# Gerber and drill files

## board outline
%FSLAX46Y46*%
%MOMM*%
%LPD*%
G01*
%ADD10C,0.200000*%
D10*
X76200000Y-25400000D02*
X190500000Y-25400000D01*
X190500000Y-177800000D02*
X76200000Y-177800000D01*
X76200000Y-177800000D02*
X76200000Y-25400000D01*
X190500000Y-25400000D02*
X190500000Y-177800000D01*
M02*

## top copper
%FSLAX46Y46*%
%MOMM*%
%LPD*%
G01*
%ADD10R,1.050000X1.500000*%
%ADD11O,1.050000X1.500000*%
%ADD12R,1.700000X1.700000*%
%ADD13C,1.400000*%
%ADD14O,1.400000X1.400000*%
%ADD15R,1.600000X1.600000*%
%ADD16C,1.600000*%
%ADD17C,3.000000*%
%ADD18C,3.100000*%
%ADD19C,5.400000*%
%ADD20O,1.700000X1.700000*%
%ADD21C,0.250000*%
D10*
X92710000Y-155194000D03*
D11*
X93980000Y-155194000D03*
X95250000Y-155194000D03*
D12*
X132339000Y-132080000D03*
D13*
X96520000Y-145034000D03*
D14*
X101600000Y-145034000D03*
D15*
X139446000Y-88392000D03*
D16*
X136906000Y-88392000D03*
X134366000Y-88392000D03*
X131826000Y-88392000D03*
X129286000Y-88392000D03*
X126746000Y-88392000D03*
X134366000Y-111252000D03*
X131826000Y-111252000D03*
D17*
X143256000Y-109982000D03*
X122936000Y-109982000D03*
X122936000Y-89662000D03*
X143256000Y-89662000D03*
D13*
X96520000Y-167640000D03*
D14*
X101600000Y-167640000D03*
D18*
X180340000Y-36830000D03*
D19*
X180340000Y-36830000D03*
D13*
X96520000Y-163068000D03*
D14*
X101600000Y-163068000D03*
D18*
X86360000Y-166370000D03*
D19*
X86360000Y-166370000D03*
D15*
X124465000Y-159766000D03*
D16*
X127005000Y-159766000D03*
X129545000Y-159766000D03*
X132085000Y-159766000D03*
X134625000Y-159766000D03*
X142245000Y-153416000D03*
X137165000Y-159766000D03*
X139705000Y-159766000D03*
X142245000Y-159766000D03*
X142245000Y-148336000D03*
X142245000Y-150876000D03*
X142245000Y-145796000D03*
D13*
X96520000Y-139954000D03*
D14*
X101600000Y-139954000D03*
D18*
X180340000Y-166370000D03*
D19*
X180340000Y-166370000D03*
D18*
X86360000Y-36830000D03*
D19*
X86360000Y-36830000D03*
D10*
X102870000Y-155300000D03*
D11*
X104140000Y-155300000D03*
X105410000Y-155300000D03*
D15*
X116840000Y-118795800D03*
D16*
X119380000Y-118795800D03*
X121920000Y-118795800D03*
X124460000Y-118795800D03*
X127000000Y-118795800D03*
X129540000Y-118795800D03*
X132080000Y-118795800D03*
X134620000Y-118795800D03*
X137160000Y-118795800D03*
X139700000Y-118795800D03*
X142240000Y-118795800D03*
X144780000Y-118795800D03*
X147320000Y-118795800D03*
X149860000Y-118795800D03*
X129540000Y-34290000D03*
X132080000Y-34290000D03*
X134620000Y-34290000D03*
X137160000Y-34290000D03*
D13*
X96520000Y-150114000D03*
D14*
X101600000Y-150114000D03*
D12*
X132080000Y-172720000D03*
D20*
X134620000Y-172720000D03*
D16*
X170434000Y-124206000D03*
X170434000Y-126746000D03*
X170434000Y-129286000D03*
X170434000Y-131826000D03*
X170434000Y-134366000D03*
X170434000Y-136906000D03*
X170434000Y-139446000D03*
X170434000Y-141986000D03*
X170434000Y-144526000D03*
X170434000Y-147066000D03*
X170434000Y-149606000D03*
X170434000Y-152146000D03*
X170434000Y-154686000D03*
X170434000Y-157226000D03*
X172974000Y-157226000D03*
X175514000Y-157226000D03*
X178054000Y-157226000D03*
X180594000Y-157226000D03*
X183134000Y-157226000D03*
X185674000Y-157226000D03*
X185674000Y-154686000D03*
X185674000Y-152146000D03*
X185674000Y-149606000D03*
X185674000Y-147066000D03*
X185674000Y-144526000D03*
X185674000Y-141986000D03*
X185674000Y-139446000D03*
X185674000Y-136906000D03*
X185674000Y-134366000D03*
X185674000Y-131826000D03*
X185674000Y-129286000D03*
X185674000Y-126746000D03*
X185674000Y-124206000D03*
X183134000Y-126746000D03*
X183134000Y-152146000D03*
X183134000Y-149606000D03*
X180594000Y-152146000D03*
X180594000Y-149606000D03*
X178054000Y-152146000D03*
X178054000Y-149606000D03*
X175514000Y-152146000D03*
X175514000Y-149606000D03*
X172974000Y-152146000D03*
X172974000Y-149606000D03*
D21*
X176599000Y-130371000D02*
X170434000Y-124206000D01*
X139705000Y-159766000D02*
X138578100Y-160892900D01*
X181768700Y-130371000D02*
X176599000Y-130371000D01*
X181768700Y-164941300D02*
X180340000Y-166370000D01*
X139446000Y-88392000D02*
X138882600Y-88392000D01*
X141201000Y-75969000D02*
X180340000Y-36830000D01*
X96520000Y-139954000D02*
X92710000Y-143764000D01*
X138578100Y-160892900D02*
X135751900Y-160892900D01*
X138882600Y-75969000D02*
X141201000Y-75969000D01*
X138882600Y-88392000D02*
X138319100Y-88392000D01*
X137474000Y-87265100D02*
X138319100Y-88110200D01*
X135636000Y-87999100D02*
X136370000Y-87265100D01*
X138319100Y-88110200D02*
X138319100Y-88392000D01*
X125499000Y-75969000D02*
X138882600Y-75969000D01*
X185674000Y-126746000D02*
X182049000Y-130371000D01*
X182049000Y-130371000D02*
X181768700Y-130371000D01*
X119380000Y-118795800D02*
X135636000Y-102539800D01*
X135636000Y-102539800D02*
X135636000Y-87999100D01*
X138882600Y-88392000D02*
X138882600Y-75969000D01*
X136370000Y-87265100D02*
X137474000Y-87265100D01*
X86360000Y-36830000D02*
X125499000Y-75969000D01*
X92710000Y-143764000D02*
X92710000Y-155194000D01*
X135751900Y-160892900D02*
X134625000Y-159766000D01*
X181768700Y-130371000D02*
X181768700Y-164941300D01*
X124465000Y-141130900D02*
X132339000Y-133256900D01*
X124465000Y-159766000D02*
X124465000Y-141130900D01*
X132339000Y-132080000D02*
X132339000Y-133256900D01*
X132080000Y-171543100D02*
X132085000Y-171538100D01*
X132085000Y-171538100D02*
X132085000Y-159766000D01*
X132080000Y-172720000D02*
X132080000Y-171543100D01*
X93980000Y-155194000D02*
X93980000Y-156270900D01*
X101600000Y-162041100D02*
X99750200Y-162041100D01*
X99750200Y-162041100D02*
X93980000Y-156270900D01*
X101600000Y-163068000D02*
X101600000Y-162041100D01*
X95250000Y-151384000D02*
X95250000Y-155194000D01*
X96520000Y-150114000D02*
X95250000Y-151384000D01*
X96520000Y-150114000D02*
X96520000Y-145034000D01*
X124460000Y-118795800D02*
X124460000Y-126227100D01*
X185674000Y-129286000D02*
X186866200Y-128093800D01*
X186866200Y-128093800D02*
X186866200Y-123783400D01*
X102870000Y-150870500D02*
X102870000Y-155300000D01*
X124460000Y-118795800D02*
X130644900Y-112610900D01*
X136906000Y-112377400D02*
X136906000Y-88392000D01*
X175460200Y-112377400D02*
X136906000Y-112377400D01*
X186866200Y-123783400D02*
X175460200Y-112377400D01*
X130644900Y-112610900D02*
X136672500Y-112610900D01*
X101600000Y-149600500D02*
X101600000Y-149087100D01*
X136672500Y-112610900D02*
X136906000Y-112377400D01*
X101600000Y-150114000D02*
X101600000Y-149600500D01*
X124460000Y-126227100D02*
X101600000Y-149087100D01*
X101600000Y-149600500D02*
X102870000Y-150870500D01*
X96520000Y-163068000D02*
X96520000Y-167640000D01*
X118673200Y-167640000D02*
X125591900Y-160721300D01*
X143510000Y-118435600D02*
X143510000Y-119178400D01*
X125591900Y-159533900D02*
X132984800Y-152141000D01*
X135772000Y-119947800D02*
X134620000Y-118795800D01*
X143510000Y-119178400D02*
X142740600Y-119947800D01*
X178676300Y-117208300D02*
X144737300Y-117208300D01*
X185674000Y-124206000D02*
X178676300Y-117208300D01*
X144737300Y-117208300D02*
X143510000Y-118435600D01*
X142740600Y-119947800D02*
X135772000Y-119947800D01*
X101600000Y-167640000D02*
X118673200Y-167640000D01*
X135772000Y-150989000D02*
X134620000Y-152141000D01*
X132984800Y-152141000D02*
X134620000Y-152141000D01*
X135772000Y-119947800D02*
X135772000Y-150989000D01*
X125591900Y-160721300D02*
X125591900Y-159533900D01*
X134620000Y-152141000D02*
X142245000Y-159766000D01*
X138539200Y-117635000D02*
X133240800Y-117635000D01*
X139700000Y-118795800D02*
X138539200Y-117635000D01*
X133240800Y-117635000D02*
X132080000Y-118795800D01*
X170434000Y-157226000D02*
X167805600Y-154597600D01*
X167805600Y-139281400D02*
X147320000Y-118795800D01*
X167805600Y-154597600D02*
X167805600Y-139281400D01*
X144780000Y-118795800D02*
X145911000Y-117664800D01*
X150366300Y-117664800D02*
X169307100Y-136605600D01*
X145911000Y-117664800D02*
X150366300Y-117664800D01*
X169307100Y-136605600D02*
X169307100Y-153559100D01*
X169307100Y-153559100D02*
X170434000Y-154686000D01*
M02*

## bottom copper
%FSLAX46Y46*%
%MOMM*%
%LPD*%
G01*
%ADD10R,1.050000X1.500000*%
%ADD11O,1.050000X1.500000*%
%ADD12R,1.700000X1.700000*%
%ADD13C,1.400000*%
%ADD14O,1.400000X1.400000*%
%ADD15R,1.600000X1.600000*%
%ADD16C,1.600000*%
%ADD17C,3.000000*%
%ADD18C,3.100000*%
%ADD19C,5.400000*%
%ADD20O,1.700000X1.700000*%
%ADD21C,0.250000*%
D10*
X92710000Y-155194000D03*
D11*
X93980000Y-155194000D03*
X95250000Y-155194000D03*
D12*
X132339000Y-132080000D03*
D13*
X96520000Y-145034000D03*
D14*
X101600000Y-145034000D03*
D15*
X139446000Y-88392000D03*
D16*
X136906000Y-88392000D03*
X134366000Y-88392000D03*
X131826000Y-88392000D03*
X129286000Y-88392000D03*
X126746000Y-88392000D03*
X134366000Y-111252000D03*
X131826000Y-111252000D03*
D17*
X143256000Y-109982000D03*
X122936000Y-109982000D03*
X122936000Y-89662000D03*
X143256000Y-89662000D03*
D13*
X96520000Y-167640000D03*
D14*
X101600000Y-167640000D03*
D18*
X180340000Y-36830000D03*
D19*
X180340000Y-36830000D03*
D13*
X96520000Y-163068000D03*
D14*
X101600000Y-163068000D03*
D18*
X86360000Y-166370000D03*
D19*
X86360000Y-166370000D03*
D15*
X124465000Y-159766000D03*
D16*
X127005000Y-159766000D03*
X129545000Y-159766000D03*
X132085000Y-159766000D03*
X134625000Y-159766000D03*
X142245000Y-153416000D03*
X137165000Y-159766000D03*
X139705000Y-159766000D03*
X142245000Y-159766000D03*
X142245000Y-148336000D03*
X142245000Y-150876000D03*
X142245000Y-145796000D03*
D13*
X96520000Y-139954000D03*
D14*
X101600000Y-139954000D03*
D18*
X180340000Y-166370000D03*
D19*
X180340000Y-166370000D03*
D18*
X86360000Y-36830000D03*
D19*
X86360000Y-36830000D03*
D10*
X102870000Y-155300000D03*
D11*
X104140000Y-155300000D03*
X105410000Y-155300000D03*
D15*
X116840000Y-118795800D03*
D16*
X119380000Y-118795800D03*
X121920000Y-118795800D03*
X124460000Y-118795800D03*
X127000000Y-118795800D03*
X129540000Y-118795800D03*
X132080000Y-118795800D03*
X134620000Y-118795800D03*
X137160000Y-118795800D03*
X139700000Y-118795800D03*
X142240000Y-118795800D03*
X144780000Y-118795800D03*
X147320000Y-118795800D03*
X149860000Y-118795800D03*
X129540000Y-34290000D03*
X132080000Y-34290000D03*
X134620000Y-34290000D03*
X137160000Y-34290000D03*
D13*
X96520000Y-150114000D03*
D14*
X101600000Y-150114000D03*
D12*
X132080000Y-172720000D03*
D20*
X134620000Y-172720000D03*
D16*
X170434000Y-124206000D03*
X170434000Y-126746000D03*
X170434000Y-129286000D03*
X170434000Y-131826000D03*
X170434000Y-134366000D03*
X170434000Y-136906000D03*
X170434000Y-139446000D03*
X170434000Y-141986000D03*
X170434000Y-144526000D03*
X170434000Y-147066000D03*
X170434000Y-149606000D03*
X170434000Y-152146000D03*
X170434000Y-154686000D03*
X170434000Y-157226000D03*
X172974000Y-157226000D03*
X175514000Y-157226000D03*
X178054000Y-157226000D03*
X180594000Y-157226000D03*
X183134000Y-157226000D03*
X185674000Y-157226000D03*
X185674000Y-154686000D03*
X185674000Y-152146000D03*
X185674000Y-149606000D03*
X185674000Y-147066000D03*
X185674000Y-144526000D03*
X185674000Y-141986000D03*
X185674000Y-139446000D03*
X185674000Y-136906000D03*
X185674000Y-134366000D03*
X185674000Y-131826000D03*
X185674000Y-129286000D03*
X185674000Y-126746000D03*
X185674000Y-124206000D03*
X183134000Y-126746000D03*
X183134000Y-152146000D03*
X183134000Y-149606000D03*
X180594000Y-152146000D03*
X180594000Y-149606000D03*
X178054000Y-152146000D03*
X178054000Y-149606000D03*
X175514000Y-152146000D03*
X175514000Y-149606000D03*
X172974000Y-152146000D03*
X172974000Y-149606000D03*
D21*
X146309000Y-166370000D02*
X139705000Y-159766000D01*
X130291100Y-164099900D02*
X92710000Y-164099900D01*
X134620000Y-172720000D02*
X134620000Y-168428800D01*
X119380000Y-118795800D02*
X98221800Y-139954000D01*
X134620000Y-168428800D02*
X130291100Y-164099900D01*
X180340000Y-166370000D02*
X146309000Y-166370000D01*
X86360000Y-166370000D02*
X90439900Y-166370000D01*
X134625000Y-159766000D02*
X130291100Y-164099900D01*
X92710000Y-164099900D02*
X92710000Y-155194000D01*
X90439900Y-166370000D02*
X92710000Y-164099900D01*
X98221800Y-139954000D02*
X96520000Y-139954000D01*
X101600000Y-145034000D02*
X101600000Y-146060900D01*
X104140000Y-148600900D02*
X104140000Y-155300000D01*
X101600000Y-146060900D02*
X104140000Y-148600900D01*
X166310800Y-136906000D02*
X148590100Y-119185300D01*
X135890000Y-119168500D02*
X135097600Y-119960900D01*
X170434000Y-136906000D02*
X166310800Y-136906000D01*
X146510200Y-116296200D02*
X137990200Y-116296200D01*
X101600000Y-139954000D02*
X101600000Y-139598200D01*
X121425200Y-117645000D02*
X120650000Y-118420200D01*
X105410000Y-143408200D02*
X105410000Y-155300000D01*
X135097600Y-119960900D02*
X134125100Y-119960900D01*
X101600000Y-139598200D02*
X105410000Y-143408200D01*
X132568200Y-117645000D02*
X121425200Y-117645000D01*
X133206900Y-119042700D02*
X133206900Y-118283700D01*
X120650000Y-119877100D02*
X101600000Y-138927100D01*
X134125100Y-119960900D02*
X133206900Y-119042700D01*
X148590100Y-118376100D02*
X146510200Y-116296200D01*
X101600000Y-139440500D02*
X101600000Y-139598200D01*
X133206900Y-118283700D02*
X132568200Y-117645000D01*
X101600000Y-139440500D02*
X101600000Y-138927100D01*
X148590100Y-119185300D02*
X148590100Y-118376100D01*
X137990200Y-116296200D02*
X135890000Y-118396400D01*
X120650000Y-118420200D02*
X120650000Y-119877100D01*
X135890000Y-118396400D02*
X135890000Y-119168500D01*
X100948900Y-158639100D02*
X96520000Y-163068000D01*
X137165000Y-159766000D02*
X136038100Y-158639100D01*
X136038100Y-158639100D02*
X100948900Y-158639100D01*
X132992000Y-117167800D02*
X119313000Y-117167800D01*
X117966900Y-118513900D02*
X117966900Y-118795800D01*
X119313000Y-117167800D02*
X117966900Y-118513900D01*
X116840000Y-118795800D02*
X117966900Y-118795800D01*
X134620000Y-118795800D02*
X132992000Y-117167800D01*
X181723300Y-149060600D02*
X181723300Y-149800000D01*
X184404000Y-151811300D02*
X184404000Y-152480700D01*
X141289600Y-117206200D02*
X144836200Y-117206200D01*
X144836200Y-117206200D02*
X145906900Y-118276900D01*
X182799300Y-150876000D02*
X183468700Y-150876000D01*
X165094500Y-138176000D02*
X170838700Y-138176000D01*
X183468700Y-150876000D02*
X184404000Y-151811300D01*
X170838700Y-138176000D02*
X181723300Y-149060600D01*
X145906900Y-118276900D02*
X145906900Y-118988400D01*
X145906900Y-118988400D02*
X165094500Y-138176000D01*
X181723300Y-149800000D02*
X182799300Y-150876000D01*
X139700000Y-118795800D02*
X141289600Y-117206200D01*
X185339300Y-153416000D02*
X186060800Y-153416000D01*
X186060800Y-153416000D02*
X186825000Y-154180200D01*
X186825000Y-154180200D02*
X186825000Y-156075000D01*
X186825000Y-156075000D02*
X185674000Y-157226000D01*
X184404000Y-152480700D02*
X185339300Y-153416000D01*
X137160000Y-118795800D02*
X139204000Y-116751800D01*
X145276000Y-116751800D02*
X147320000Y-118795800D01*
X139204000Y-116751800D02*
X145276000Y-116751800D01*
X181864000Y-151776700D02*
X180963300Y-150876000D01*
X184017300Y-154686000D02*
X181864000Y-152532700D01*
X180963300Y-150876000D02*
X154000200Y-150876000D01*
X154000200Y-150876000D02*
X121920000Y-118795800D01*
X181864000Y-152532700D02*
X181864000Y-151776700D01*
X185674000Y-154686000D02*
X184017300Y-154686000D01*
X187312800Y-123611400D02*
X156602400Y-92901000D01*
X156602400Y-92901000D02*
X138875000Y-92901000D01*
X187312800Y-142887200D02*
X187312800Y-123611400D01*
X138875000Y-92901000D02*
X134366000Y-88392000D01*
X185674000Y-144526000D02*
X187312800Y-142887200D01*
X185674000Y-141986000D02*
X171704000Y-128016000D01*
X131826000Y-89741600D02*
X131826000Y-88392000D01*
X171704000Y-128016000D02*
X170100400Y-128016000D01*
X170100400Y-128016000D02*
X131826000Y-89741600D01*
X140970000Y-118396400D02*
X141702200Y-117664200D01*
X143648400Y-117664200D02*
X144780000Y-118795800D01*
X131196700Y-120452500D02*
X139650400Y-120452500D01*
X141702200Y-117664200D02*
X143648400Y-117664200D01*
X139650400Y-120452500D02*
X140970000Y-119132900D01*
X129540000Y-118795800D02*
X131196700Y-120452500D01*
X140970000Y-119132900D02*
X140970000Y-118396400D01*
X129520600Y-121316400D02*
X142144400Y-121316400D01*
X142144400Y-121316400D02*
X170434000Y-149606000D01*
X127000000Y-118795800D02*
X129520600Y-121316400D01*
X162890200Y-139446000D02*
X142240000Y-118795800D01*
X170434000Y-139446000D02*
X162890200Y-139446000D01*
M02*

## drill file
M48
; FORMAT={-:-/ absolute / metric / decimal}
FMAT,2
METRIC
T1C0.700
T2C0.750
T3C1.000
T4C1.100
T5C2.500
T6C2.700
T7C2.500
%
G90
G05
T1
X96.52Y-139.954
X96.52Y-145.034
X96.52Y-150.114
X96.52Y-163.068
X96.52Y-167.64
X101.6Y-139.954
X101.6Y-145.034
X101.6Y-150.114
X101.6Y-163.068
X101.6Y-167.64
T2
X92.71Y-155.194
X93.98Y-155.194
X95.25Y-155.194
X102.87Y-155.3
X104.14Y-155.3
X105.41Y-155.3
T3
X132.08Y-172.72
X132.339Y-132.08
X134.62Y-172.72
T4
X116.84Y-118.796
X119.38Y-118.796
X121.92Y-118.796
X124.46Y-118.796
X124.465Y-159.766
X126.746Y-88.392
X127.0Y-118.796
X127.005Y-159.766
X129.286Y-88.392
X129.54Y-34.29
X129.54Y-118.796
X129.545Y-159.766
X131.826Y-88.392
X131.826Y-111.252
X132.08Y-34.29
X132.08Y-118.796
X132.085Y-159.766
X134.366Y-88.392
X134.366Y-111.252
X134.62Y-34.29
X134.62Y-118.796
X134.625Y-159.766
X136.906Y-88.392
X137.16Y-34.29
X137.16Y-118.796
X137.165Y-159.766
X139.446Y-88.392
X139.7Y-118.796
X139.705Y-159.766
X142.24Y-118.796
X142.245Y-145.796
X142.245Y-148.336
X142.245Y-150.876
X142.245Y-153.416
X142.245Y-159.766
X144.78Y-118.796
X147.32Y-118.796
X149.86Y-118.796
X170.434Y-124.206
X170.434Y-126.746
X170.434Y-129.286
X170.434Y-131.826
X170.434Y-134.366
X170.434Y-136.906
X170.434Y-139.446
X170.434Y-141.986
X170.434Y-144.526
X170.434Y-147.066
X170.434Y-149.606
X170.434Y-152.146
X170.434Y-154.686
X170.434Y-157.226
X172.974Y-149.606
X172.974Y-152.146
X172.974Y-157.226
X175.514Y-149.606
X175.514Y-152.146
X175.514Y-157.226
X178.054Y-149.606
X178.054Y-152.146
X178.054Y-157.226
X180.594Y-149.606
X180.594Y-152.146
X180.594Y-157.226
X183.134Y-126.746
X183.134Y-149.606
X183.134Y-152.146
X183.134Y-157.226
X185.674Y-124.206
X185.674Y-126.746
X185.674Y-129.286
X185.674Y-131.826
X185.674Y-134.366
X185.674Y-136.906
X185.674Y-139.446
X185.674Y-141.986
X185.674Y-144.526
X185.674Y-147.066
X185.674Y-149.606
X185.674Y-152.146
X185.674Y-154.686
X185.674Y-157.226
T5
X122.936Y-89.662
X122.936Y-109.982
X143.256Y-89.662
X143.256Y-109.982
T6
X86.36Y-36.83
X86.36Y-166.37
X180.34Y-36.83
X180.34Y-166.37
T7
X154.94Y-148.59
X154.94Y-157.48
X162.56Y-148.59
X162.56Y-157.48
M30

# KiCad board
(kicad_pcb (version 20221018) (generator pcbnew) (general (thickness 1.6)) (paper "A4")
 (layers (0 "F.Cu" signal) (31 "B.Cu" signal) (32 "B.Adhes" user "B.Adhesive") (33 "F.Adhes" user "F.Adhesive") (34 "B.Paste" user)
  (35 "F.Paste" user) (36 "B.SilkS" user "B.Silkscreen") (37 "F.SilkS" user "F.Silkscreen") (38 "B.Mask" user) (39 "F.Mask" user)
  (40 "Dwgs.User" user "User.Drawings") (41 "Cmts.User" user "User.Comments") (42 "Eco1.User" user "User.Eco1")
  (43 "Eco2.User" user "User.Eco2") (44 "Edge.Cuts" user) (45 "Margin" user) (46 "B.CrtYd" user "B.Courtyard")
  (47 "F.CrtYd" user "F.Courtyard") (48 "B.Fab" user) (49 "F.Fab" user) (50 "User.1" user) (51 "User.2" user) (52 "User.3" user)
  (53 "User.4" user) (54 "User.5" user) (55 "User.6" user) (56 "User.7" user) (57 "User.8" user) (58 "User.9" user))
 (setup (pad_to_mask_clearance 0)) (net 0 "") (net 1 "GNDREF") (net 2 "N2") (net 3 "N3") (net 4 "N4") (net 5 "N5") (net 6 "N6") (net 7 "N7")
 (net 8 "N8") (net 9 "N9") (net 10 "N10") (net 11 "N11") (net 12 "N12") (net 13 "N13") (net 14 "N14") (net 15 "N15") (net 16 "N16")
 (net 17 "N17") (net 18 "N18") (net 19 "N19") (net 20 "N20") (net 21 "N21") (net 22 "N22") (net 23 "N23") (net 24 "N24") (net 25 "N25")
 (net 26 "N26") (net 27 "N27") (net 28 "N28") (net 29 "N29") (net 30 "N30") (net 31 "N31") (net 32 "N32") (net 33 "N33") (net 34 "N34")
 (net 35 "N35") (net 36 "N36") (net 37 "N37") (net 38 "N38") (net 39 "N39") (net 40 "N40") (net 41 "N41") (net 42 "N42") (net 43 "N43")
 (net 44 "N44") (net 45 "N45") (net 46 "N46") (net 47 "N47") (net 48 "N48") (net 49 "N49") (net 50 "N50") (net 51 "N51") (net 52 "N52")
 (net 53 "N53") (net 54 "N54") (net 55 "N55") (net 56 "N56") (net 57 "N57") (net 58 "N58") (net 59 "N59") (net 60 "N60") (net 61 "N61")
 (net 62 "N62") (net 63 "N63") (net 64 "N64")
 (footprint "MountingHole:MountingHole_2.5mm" (layer "F.Cu") (at 154.94 157.48)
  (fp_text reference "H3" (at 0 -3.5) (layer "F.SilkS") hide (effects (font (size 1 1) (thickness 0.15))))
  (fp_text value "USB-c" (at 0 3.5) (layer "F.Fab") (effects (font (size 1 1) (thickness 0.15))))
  (pad "" np_thru_hole circle (at 0 0) (size 2.5 2.5) (drill 2.5) (layers "*.Cu" "*.Mask")))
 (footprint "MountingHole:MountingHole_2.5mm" (layer "F.Cu") (at 162.56 148.59)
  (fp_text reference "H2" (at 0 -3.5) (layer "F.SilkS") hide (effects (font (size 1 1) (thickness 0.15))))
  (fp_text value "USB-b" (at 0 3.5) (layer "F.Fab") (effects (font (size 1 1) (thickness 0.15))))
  (pad "" np_thru_hole circle (at 0 0) (size 2.5 2.5) (drill 2.5) (layers "*.Cu" "*.Mask")))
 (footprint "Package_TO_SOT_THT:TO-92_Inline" (layer "F.Cu") (at 92.71 155.194)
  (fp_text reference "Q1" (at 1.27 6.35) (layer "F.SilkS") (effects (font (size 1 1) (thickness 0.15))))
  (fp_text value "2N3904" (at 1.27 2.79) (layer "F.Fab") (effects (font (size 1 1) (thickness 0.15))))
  (pad "1" thru_hole rect (at 0 0) (size 1.05 1.5) (drill 0.75) (layers "*.Cu" "*.Mask") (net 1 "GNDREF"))
  (pad "2" thru_hole oval (at 1.27 0) (size 1.05 1.5) (drill 0.75) (layers "*.Cu" "*.Mask") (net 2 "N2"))
  (pad "3" thru_hole oval (at 2.54 0) (size 1.05 1.5) (drill 0.75) (layers "*.Cu" "*.Mask") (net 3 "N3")))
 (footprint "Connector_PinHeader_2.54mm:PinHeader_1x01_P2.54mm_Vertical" (layer "F.Cu") (at 132.339 132.08)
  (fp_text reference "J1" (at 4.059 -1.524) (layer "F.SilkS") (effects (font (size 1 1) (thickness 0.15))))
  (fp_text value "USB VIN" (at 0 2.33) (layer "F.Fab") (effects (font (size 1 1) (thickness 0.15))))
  (pad "1" thru_hole rect (at 0 0) (size 1.7 1.7) (drill 1) (layers "*.Cu" "*.Mask") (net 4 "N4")))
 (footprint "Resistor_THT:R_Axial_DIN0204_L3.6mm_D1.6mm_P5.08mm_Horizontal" (layer "F.Cu") (at 96.52 145.034)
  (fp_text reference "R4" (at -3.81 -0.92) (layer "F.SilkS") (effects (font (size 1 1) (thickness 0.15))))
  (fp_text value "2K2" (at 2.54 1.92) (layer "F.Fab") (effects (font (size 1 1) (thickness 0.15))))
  (pad "1" thru_hole circle (at 0 0) (size 1.4 1.4) (drill 0.7) (layers "*.Cu" "*.Mask") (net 3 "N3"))
  (pad "2" thru_hole oval (at 5.08 0) (size 1.4 1.4) (drill 0.7) (layers "*.Cu" "*.Mask") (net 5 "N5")))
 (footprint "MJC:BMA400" (layer "F.Cu") (at 133.096 99.822 180)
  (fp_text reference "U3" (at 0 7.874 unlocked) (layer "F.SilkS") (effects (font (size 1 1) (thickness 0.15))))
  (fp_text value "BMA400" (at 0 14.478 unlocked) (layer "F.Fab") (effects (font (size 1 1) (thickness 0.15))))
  (pad "1" thru_hole rect (at -6.35 11.43 180) (size 1.6 1.6) (drill 1.1) (layers "*.Cu" "*.Mask") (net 1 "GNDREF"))
  (pad "2" thru_hole circle (at -3.81 11.43 180) (size 1.6 1.6) (drill 1.1) (layers "*.Cu" "*.Mask") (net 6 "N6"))
  (pad "3" thru_hole circle (at -1.27 11.43 180) (size 1.6 1.6) (drill 1.1) (layers "*.Cu" "*.Mask") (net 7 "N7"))
  (pad "4" thru_hole circle (at 1.27 11.43 180) (size 1.6 1.6) (drill 1.1) (layers "*.Cu" "*.Mask") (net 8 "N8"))
  (pad "5" thru_hole circle (at 3.81 11.43 180) (size 1.6 1.6) (drill 1.1) (layers "*.Cu" "*.Mask") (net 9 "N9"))
  (pad "6" thru_hole circle (at 6.35 11.43 180) (size 1.6 1.6) (drill 1.1) (layers "*.Cu" "*.Mask") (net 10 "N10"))
  (pad "7" thru_hole circle (at -1.27 -11.43 180) (size 1.6 1.6) (drill 1.1) (layers "*.Cu" "*.Mask") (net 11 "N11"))
  (pad "8" thru_hole circle (at 1.27 -11.43 180) (size 1.6 1.6) (drill 1.1) (layers "*.Cu" "*.Mask") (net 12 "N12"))
  (pad "9" thru_hole circle (at -10.16 -10.16 180) (size 3 3) (drill 2.5) (layers "*.Cu" "*.Mask"))
  (pad "10" thru_hole circle (at 10.16 -10.16 180) (size 3 3) (drill 2.5) (layers "*.Cu" "*.Mask"))
  (pad "11" thru_hole circle (at 10.16 10.16 180) (size 3 3) (drill 2.5) (layers "*.Cu" "*.Mask"))
  (pad "12" thru_hole circle (at -10.16 10.16 180) (size 3 3) (drill 2.5) (layers "*.Cu" "*.Mask")))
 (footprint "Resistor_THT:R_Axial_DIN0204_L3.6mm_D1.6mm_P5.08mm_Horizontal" (layer "F.Cu") (at 96.52 167.64)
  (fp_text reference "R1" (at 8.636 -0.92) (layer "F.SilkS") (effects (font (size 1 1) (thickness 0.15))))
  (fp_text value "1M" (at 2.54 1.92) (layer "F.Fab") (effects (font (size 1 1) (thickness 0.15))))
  (pad "1" thru_hole circle (at 0 0) (size 1.4 1.4) (drill 0.7) (layers "*.Cu" "*.Mask") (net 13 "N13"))
  (pad "2" thru_hole oval (at 5.08 0) (size 1.4 1.4) (drill 0.7) (layers "*.Cu" "*.Mask") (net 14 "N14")))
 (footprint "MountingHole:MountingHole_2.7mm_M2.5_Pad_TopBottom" (layer "F.Cu") (at 180.34 36.83)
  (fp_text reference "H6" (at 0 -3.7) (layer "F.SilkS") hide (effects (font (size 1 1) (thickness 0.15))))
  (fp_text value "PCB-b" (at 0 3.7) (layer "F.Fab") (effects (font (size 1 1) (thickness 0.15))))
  (pad "1" thru_hole circle (at 0 0) (size 3.1 3.1) (drill 2.7) (layers "*.Cu" "*.Mask") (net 1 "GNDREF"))
  (pad "1" connect circle (at 0 0) (size 5.4 5.4) (layers "F.Cu" "F.Mask") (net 1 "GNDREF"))
  (pad "1" connect circle (at 0 0) (size 5.4 5.4) (layers "B.Cu" "B.Mask") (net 1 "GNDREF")))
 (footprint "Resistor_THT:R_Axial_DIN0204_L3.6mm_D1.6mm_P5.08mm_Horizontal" (layer "F.Cu") (at 96.52 163.068)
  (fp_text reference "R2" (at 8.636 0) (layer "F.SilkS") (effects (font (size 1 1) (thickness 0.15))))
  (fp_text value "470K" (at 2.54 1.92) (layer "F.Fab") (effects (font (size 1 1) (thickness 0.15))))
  (pad "1" thru_hole circle (at 0 0) (size 1.4 1.4) (drill 0.7) (layers "*.Cu" "*.Mask") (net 13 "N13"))
  (pad "2" thru_hole oval (at 5.08 0) (size 1.4 1.4) (drill 0.7) (layers "*.Cu" "*.Mask") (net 2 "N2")))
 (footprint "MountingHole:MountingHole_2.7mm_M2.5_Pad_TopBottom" (layer "F.Cu") (at 86.36 166.37)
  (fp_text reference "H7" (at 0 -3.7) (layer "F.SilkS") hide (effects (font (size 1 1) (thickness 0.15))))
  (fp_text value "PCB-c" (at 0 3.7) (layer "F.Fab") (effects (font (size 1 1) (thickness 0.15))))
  (pad "1" thru_hole circle (at 0 0) (size 3.1 3.1) (drill 2.7) (layers "*.Cu" "*.Mask") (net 1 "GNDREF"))
  (pad "1" connect circle (at 0 0) (size 5.4 5.4) (layers "F.Cu" "F.Mask") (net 1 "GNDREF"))
  (pad "1" connect circle (at 0 0) (size 5.4 5.4) (layers "B.Cu" "B.Mask") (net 1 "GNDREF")))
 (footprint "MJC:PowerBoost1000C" (layer "F.Cu") (at 129.545 149.606 90)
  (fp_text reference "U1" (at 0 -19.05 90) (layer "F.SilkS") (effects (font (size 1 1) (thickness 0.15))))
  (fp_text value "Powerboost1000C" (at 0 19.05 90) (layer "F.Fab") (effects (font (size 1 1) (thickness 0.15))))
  (pad "1" thru_hole rect (at -10.16 -5.08 90) (size 1.6 1.6) (drill 1.1) (layers "*.Cu" "*.Mask") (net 4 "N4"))
  (pad "2" thru_hole circle (at -10.16 -2.54 90) (size 1.6 1.6) (drill 1.1) (layers "*.Cu" "*.Mask") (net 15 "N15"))
  (pad "3" thru_hole circle (at -10.16 0 90) (size 1.6 1.6) (drill 1.1) (layers "*.Cu" "*.Mask") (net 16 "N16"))
  (pad "4" thru_hole circle (at -10.16 2.54 90) (size 1.6 1.6) (drill 1.1) (layers "*.Cu" "*.Mask") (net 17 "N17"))
  (pad "5" thru_hole circle (at -10.16 5.08 90) (size 1.6 1.6) (drill 1.1) (layers "*.Cu" "*.Mask") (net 1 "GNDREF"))
  (pad "5V" thru_hole circle (at -3.81 12.7 90) (size 1.6 1.6) (drill 1.1) (layers "*.Cu" "*.Mask") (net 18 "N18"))
  (pad "6" thru_hole circle (at -10.16 7.62 90) (size 1.6 1.6) (drill 1.1) (layers "*.Cu" "*.Mask") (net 13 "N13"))
  (pad "7" thru_hole circle (at -10.16 10.16 90) (size 1.6 1.6) (drill 1.1) (layers "*.Cu" "*.Mask") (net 1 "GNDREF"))
  (pad "8" thru_hole circle (at -10.16 12.7 90) (size 1.6 1.6) (drill 1.1) (layers "*.Cu" "*.Mask") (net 14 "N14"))
  (pad "D+" thru_hole circle (at 1.27 12.7 90) (size 1.6 1.6) (drill 1.1) (layers "*.Cu" "*.Mask") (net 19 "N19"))
  (pad "D-" thru_hole circle (at -1.27 12.7 90) (size 1.6 1.6) (drill 1.1) (layers "*.Cu" "*.Mask") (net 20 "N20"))
  (pad "UG" thru_hole circle (at 3.81 12.7 90) (size 1.6 1.6) (drill 1.1) (layers "*.Cu" "*.Mask") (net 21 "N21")))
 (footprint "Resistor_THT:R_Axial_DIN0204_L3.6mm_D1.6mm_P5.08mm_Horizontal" (layer "F.Cu") (at 96.52 139.954)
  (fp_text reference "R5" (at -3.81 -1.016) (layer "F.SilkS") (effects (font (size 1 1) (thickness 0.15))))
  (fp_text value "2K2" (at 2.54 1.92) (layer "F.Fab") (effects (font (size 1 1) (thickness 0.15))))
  (pad "1" thru_hole circle (at 0 0) (size 1.4 1.4) (drill 0.7) (layers "*.Cu" "*.Mask") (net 1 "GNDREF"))
  (pad "2" thru_hole oval (at 5.08 0) (size 1.4 1.4) (drill 0.7) (layers "*.Cu" "*.Mask") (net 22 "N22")))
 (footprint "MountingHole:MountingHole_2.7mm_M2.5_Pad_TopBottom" (layer "F.Cu") (at 180.34 166.37)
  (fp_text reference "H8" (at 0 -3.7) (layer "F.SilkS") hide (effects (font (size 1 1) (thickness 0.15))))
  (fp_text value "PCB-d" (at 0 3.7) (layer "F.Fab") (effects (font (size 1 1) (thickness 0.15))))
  (pad "1" thru_hole circle (at 0 0) (size 3.1 3.1) (drill 2.7) (layers "*.Cu" "*.Mask") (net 1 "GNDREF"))
  (pad "1" connect circle (at 0 0) (size 5.4 5.4) (layers "F.Cu" "F.Mask") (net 1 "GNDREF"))
  (pad "1" connect circle (at 0 0) (size 5.4 5.4) (layers "B.Cu" "B.Mask") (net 1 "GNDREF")))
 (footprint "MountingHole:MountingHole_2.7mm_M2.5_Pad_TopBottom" (layer "F.Cu") (at 86.36 36.83)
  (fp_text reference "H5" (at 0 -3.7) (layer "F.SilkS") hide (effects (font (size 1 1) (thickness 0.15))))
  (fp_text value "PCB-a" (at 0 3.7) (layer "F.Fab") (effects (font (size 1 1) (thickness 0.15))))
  (pad "1" thru_hole circle (at 0 0) (size 3.1 3.1) (drill 2.7) (layers "*.Cu" "*.Mask") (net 1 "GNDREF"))
  (pad "1" connect circle (at 0 0) (size 5.4 5.4) (layers "F.Cu" "F.Mask") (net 1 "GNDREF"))
  (pad "1" connect circle (at 0 0) (size 5.4 5.4) (layers "B.Cu" "B.Mask") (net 1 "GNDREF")))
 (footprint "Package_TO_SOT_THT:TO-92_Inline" (layer "F.Cu") (at 102.87 155.3)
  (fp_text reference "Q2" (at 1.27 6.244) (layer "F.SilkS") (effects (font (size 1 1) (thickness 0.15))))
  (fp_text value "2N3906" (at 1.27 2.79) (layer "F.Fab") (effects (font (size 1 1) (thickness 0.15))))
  (pad "1" thru_hole rect (at 0 0) (size 1.05 1.5) (drill 0.75) (layers "*.Cu" "*.Mask") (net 6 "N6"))
  (pad "2" thru_hole oval (at 1.27 0) (size 1.05 1.5) (drill 0.75) (layers "*.Cu" "*.Mask") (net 5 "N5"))
  (pad "3" thru_hole oval (at 2.54 0) (size 1.05 1.5) (drill 0.75) (layers "*.Cu" "*.Mask") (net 22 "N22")))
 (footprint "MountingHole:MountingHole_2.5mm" (layer "F.Cu") (at 154.94 148.59)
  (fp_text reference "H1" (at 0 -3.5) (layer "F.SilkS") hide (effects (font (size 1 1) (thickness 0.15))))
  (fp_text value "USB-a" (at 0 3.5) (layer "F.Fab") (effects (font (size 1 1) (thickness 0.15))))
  (pad "" np_thru_hole circle (at 0 0) (size 2.5 2.5) (drill 2.5) (layers "*.Cu" "*.Mask")))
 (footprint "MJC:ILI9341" (layer "F.Cu") (at 133.35 76.0476)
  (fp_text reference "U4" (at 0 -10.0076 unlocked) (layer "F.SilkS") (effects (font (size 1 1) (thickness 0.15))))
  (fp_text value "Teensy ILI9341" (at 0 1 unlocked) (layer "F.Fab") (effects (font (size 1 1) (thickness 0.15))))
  (pad "1" thru_hole rect (at -16.51 42.7482) (size 1.6 1.6) (drill 1.1) (layers "*.Cu" "*.Mask") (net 14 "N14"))
  (pad "2" thru_hole circle (at -13.97 42.7482) (size 1.6 1.6) (drill 1.1) (layers "*.Cu" "*.Mask") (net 1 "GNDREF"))
  (pad "3" thru_hole circle (at -11.43 42.7482) (size 1.6 1.6) (drill 1.1) (layers "*.Cu" "*.Mask") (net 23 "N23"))
  (pad "4" thru_hole circle (at -8.89 42.7482) (size 1.6 1.6) (drill 1.1) (layers "*.Cu" "*.Mask") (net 6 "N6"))
  (pad "5" thru_hole circle (at -6.35 42.7482) (size 1.6 1.6) (drill 1.1) (layers "*.Cu" "*.Mask") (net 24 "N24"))
  (pad "6" thru_hole circle (at -3.81 42.7482) (size 1.6 1.6) (drill 1.1) (layers "*.Cu" "*.Mask") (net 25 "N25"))
  (pad "7" thru_hole circle (at -1.27 42.7482) (size 1.6 1.6) (drill 1.1) (layers "*.Cu" "*.Mask") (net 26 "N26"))
  (pad "8" thru_hole circle (at 1.27 42.7482) (size 1.6 1.6) (drill 1.1) (layers "*.Cu" "*.Mask") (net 14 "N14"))
  (pad "9" thru_hole circle (at 3.81 42.7482) (size 1.6 1.6) (drill 1.1) (layers "*.Cu" "*.Mask") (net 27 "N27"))
  (pad "10" thru_hole circle (at 6.35 42.7482) (size 1.6 1.6) (drill 1.1) (layers "*.Cu" "*.Mask") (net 26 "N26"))
  (pad "11" thru_hole circle (at 8.89 42.7482) (size 1.6 1.6) (drill 1.1) (layers "*.Cu" "*.Mask") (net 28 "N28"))
  (pad "12" thru_hole circle (at 11.43 42.7482) (size 1.6 1.6) (drill 1.1) (layers "*.Cu" "*.Mask") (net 25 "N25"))
  (pad "13" thru_hole circle (at 13.97 42.7482) (size 1.6 1.6) (drill 1.1) (layers "*.Cu" "*.Mask") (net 27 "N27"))
  (pad "14" thru_hole circle (at 16.51 42.7482) (size 1.6 1.6) (drill 1.1) (layers "*.Cu" "*.Mask") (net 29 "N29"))
  (pad "15" thru_hole circle (at -3.81 -41.7576) (size 1.6 1.6) (drill 1.1) (layers "*.Cu" "*.Mask") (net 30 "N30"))
  (pad "16" thru_hole circle (at -1.27 -41.7576) (size 1.6 1.6) (drill 1.1) (layers "*.Cu" "*.Mask") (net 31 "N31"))
  (pad "17" thru_hole circle (at 1.27 -41.7576) (size 1.6 1.6) (drill 1.1) (layers "*.Cu" "*.Mask") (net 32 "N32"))
  (pad "18" thru_hole circle (at 3.81 -41.7576) (size 1.6 1.6) (drill 1.1) (layers "*.Cu" "*.Mask") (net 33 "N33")))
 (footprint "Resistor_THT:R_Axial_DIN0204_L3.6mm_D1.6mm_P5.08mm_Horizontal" (layer "F.Cu") (at 96.52 150.114)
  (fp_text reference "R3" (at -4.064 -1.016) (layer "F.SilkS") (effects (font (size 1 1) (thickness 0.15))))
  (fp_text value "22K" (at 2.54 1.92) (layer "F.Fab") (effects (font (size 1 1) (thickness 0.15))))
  (pad "1" thru_hole circle (at 0 0) (size 1.4 1.4) (drill 0.7) (layers "*.Cu" "*.Mask") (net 3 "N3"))
  (pad "2" thru_hole oval (at 5.08 0) (size 1.4 1.4) (drill 0.7) (layers "*.Cu" "*.Mask") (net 6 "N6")))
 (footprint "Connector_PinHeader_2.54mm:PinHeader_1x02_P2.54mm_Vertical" (layer "F.Cu") (at 132.08 172.72 90)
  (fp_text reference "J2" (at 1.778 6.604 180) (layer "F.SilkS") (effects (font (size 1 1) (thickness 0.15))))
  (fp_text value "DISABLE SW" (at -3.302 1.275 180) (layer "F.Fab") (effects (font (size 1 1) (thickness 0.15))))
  (pad "1" thru_hole rect (at 0 0 90) (size 1.7 1.7) (drill 1) (layers "*.Cu" "*.Mask") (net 17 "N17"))
  (pad "2" thru_hole oval (at 0 2.54 90) (size 1.7 1.7) (drill 1) (layers "*.Cu" "*.Mask") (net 1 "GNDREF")))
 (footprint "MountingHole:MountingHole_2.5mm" (layer "F.Cu") (at 162.56 157.48)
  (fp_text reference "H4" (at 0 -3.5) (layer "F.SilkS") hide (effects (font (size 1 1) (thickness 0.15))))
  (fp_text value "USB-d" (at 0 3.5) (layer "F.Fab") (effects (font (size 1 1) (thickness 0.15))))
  (pad "" np_thru_hole circle (at 0 0) (size 2.5 2.5) (drill 2.5) (layers "*.Cu" "*.Mask")))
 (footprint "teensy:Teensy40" (layer "F.Cu") (at 178.054 140.716 -90)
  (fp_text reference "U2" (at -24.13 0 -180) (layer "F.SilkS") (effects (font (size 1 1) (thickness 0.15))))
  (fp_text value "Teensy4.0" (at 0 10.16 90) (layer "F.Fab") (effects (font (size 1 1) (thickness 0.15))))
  (pad "1" thru_hole circle (at -16.51 7.62 270) (size 1.6 1.6) (drill 1.1) (layers "*.Cu" "*.Mask") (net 1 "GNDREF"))
  (pad "2" thru_hole circle (at -13.97 7.62 270) (size 1.6 1.6) (drill 1.1) (layers "*.Cu" "*.Mask") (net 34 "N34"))
  (pad "3" thru_hole circle (at -11.43 7.62 270) (size 1.6 1.6) (drill 1.1) (layers "*.Cu" "*.Mask") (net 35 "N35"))
  (pad "4" thru_hole circle (at -8.89 7.62 270) (size 1.6 1.6) (drill 1.1) (layers "*.Cu" "*.Mask") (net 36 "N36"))
  (pad "5" thru_hole circle (at -6.35 7.62 270) (size 1.6 1.6) (drill 1.1) (layers "*.Cu" "*.Mask") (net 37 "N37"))
  (pad "6" thru_hole circle (at -3.81 7.62 270) (size 1.6 1.6) (drill 1.1) (layers "*.Cu" "*.Mask") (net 22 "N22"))
  (pad "7" thru_hole circle (at -1.27 7.62 270) (size 1.6 1.6) (drill 1.1) (layers "*.Cu" "*.Mask") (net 28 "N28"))
  (pad "8" thru_hole circle (at 1.27 7.62 270) (size 1.6 1.6) (drill 1.1) (layers "*.Cu" "*.Mask") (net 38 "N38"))
  (pad "9" thru_hole circle (at 3.81 7.62 270) (size 1.6 1.6) (drill 1.1) (layers "*.Cu" "*.Mask") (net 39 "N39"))
  (pad "10" thru_hole circle (at 6.35 7.62 270) (size 1.6 1.6) (drill 1.1) (layers "*.Cu" "*.Mask") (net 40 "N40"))
  (pad "11" thru_hole circle (at 8.89 7.62 270) (size 1.6 1.6) (drill 1.1) (layers "*.Cu" "*.Mask") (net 24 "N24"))
  (pad "12" thru_hole circle (at 11.43 7.62 270) (size 1.6 1.6) (drill 1.1) (layers "*.Cu" "*.Mask") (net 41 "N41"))
  (pad "13" thru_hole circle (at 13.97 7.62 270) (size 1.6 1.6) (drill 1.1) (layers "*.Cu" "*.Mask") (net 25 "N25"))
  (pad "14" thru_hole circle (at 16.51 7.62 270) (size 1.6 1.6) (drill 1.1) (layers "*.Cu" "*.Mask") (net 27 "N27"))
  (pad "15" thru_hole circle (at 16.51 5.08 270) (size 1.6 1.6) (drill 1.1) (layers "*.Cu" "*.Mask") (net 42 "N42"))
  (pad "16" thru_hole circle (at 16.51 2.54 270) (size 1.6 1.6) (drill 1.1) (layers "*.Cu" "*.Mask") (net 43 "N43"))
  (pad "17" thru_hole circle (at 16.51 0 270) (size 1.6 1.6) (drill 1.1) (layers "*.Cu" "*.Mask") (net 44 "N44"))
  (pad "18" thru_hole circle (at 16.51 -2.54 270) (size 1.6 1.6) (drill 1.1) (layers "*.Cu" "*.Mask") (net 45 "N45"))
  (pad "19" thru_hole circle (at 16.51 -5.08 270) (size 1.6 1.6) (drill 1.1) (layers "*.Cu" "*.Mask") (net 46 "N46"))
  (pad "20" thru_hole circle (at 16.51 -7.62 270) (size 1.6 1.6) (drill 1.1) (layers "*.Cu" "*.Mask") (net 26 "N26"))
  (pad "21" thru_hole circle (at 13.97 -7.62 270) (size 1.6 1.6) (drill 1.1) (layers "*.Cu" "*.Mask") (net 23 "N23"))
  (pad "22" thru_hole circle (at 11.43 -7.62 270) (size 1.6 1.6) (drill 1.1) (layers "*.Cu" "*.Mask") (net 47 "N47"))
  (pad "23" thru_hole circle (at 8.89 -7.62 270) (size 1.6 1.6) (drill 1.1) (layers "*.Cu" "*.Mask") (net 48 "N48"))
  (pad "24" thru_hole circle (at 6.35 -7.62 270) (size 1.6 1.6) (drill 1.1) (layers "*.Cu" "*.Mask") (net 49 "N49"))
  (pad "25" thru_hole circle (at 3.81 -7.62 270) (size 1.6 1.6) (drill 1.1) (layers "*.Cu" "*.Mask") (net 7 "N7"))
  (pad "26" thru_hole circle (at 1.27 -7.62 270) (size 1.6 1.6) (drill 1.1) (layers "*.Cu" "*.Mask") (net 8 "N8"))
  (pad "27" thru_hole circle (at -1.27 -7.62 270) (size 1.6 1.6) (drill 1.1) (layers "*.Cu" "*.Mask") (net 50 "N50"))
  (pad "28" thru_hole circle (at -3.81 -7.62 270) (size 1.6 1.6) (drill 1.1) (layers "*.Cu" "*.Mask") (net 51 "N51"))
  (pad "29" thru_hole circle (at -6.35 -7.62 270) (size 1.6 1.6) (drill 1.1) (layers "*.Cu" "*.Mask") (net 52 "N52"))
  (pad "30" thru_hole circle (at -8.89 -7.62 270) (size 1.6 1.6) (drill 1.1) (layers "*.Cu" "*.Mask") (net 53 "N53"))
  (pad "31" thru_hole circle (at -11.43 -7.62 270) (size 1.6 1.6) (drill 1.1) (layers "*.Cu" "*.Mask") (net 6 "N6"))
  (pad "32" thru_hole circle (at -13.97 -7.62 270) (size 1.6 1.6) (drill 1.1) (layers "*.Cu" "*.Mask") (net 1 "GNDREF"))
  (pad "33" thru_hole circle (at -16.51 -7.62 270) (size 1.6 1.6) (drill 1.1) (layers "*.Cu" "*.Mask") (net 14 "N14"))
  (pad "34" thru_hole circle (at -13.97 -5.08 270) (size 1.6 1.6) (drill 1.1) (layers "*.Cu" "*.Mask") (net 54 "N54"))
  (pad "35" thru_hole circle (at 11.43 -5.08 270) (size 1.6 1.6) (drill 1.1) (layers "*.Cu" "*.Mask") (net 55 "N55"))
  (pad "36" thru_hole circle (at 8.89 -5.08 270) (size 1.6 1.6) (drill 1.1) (layers "*.Cu" "*.Mask") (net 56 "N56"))
  (pad "37" thru_hole circle (at 11.43 -2.54 270) (size 1.6 1.6) (drill 1.1) (layers "*.Cu" "*.Mask") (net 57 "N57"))
  (pad "38" thru_hole circle (at 8.89 -2.54 270) (size 1.6 1.6) (drill 1.1) (layers "*.Cu" "*.Mask") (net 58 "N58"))
  (pad "39" thru_hole circle (at 11.43 0 270) (size 1.6 1.6) (drill 1.1) (layers "*.Cu" "*.Mask") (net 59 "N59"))
  (pad "40" thru_hole circle (at 8.89 0 270) (size 1.6 1.6) (drill 1.1) (layers "*.Cu" "*.Mask") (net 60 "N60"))
  (pad "41" thru_hole circle (at 11.43 2.54 270) (size 1.6 1.6) (drill 1.1) (layers "*.Cu" "*.Mask") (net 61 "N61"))
  (pad "42" thru_hole circle (at 8.89 2.54 270) (size 1.6 1.6) (drill 1.1) (layers "*.Cu" "*.Mask") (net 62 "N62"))
  (pad "43" thru_hole circle (at 11.43 5.08 270) (size 1.6 1.6) (drill 1.1) (layers "*.Cu" "*.Mask") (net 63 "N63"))
  (pad "44" thru_hole circle (at 8.89 5.08 270) (size 1.6 1.6) (drill 1.1) (layers "*.Cu" "*.Mask") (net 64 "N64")))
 (gr_line (start 76.2 25.4) (end 190.5 25.4) (stroke (width 0.2) (type default)) (layer "Edge.Cuts"))
 (gr_line (start 190.5 177.8) (end 76.2 177.8) (stroke (width 0.2) (type default)) (layer "Edge.Cuts"))
 (gr_line (start 76.2 177.8) (end 76.2 25.4) (stroke (width 0.2) (type default)) (layer "Edge.Cuts"))
 (gr_line (start 190.5 25.4) (end 190.5 177.8) (stroke (width 0.2) (type default)) (layer "Edge.Cuts"))
 (segment (start 176.599 130.371) (end 170.434 124.206) (width 0.25) (layer "F.Cu") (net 1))
 (segment (start 139.705 159.766) (end 138.5781 160.8929) (width 0.25) (layer "F.Cu") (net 1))
 (segment (start 181.7687 130.371) (end 176.599 130.371) (width 0.25) (layer "F.Cu") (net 1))
 (segment (start 181.7687 164.9413) (end 180.34 166.37) (width 0.25) (layer "F.Cu") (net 1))
 (segment (start 139.446 88.392) (end 138.8826 88.392) (width 0.25) (layer "F.Cu") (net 1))
 (segment (start 141.201 75.969) (end 180.34 36.83) (width 0.25) (layer "F.Cu") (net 1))
 (segment (start 96.52 139.954) (end 92.71 143.764) (width 0.25) (layer "F.Cu") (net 1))
 (segment (start 138.5781 160.8929) (end 135.7519 160.8929) (width 0.25) (layer "F.Cu") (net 1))
 (segment (start 138.8826 75.969) (end 141.201 75.969) (width 0.25) (layer "F.Cu") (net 1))
 (segment (start 138.8826 88.392) (end 138.3191 88.392) (width 0.25) (layer "F.Cu") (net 1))
 (segment (start 137.474 87.2651) (end 138.3191 88.1102) (width 0.25) (layer "F.Cu") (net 1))
 (segment (start 135.636 87.9991) (end 136.37 87.2651) (width 0.25) (layer "F.Cu") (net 1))
 (segment (start 138.3191 88.1102) (end 138.3191 88.392) (width 0.25) (layer "F.Cu") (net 1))
 (segment (start 125.499 75.969) (end 138.8826 75.969) (width 0.25) (layer "F.Cu") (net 1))
 (segment (start 185.674 126.746) (end 182.049 130.371) (width 0.25) (layer "F.Cu") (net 1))
 (segment (start 182.049 130.371) (end 181.7687 130.371) (width 0.25) (layer "F.Cu") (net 1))
 (segment (start 119.38 118.7958) (end 135.636 102.5398) (width 0.25) (layer "F.Cu") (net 1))
 (segment (start 135.636 102.5398) (end 135.636 87.9991) (width 0.25) (layer "F.Cu") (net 1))
 (segment (start 138.8826 88.392) (end 138.8826 75.969) (width 0.25) (layer "F.Cu") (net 1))
 (segment (start 136.37 87.2651) (end 137.474 87.2651) (width 0.25) (layer "F.Cu") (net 1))
 (segment (start 86.36 36.83) (end 125.499 75.969) (width 0.25) (layer "F.Cu") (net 1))
 (segment (start 92.71 143.764) (end 92.71 155.194) (width 0.25) (layer "F.Cu") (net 1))
 (segment (start 135.7519 160.8929) (end 134.625 159.766) (width 0.25) (layer "F.Cu") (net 1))
 (segment (start 181.7687 130.371) (end 181.7687 164.9413) (width 0.25) (layer "F.Cu") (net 1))
 (segment (start 146.309 166.37) (end 139.705 159.766) (width 0.25) (layer "B.Cu") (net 1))
 (segment (start 130.2911 164.0999) (end 92.71 164.0999) (width 0.25) (layer "B.Cu") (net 1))
 (segment (start 134.62 172.72) (end 134.62 168.4288) (width 0.25) (layer "B.Cu") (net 1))
 (segment (start 119.38 118.7958) (end 98.2218 139.954) (width 0.25) (layer "B.Cu") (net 1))
 (segment (start 134.62 168.4288) (end 130.2911 164.0999) (width 0.25) (layer "B.Cu") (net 1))
 (segment (start 180.34 166.37) (end 146.309 166.37) (width 0.25) (layer "B.Cu") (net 1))
 (segment (start 86.36 166.37) (end 90.4399 166.37) (width 0.25) (layer "B.Cu") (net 1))
 (segment (start 134.625 159.766) (end 130.2911 164.0999) (width 0.25) (layer "B.Cu") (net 1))
 (segment (start 92.71 164.0999) (end 92.71 155.194) (width 0.25) (layer "B.Cu") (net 1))
 (segment (start 90.4399 166.37) (end 92.71 164.0999) (width 0.25) (layer "B.Cu") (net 1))
 (segment (start 98.2218 139.954) (end 96.52 139.954) (width 0.25) (layer "B.Cu") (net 1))
 (segment (start 124.465 141.1309) (end 132.339 133.2569) (width 0.25) (layer "F.Cu") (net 4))
 (segment (start 124.465 159.766) (end 124.465 141.1309) (width 0.25) (layer "F.Cu") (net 4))
 (segment (start 132.339 132.08) (end 132.339 133.2569) (width 0.25) (layer "F.Cu") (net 4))
 (segment (start 132.08 171.5431) (end 132.085 171.5381) (width 0.25) (layer "F.Cu") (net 17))
 (segment (start 132.085 171.5381) (end 132.085 159.766) (width 0.25) (layer "F.Cu") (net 17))
 (segment (start 132.08 172.72) (end 132.08 171.5431) (width 0.25) (layer "F.Cu") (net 17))
 (segment (start 93.98 155.194) (end 93.98 156.2709) (width 0.25) (layer "F.Cu") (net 2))
 (segment (start 101.6 162.0411) (end 99.7502 162.0411) (width 0.25) (layer "F.Cu") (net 2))
 (segment (start 99.7502 162.0411) (end 93.98 156.2709) (width 0.25) (layer "F.Cu") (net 2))
 (segment (start 101.6 163.068) (end 101.6 162.0411) (width 0.25) (layer "F.Cu") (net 2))
 (segment (start 95.25 151.384) (end 95.25 155.194) (width 0.25) (layer "F.Cu") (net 3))
 (segment (start 96.52 150.114) (end 95.25 151.384) (width 0.25) (layer "F.Cu") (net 3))
 (segment (start 96.52 150.114) (end 96.52 145.034) (width 0.25) (layer "F.Cu") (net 3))
 (segment (start 124.46 118.7958) (end 124.46 126.2271) (width 0.25) (layer "F.Cu") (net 6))
 (segment (start 185.674 129.286) (end 186.8662 128.0938) (width 0.25) (layer "F.Cu") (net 6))
 (segment (start 186.8662 128.0938) (end 186.8662 123.7834) (width 0.25) (layer "F.Cu") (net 6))
 (segment (start 102.87 150.8705) (end 102.87 155.3) (width 0.25) (layer "F.Cu") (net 6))
 (segment (start 124.46 118.7958) (end 130.6449 112.6109) (width 0.25) (layer "F.Cu") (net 6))
 (segment (start 136.906 112.3774) (end 136.906 88.392) (width 0.25) (layer "F.Cu") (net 6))
 (segment (start 175.4602 112.3774) (end 136.906 112.3774) (width 0.25) (layer "F.Cu") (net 6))
 (segment (start 186.8662 123.7834) (end 175.4602 112.3774) (width 0.25) (layer "F.Cu") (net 6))
 (segment (start 130.6449 112.6109) (end 136.6725 112.6109) (width 0.25) (layer "F.Cu") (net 6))
 (segment (start 101.6 149.6005) (end 101.6 149.0871) (width 0.25) (layer "F.Cu") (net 6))
 (segment (start 136.6725 112.6109) (end 136.906 112.3774) (width 0.25) (layer "F.Cu") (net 6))
 (segment (start 101.6 150.114) (end 101.6 149.6005) (width 0.25) (layer "F.Cu") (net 6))
 (segment (start 124.46 126.2271) (end 101.6 149.0871) (width 0.25) (layer "F.Cu") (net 6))
 (segment (start 101.6 149.6005) (end 102.87 150.8705) (width 0.25) (layer "F.Cu") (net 6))
 (segment (start 101.6 145.034) (end 101.6 146.0609) (width 0.25) (layer "B.Cu") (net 5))
 (segment (start 104.14 148.6009) (end 104.14 155.3) (width 0.25) (layer "B.Cu") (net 5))
 (segment (start 101.6 146.0609) (end 104.14 148.6009) (width 0.25) (layer "B.Cu") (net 5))
 (segment (start 166.3108 136.906) (end 148.5901 119.1853) (width 0.25) (layer "B.Cu") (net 22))
 (segment (start 135.89 119.1685) (end 135.0976 119.9609) (width 0.25) (layer "B.Cu") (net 22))
 (segment (start 170.434 136.906) (end 166.3108 136.906) (width 0.25) (layer "B.Cu") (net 22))
 (segment (start 146.5102 116.2962) (end 137.9902 116.2962) (width 0.25) (layer "B.Cu") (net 22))
 (segment (start 101.6 139.954) (end 101.6 139.5982) (width 0.25) (layer "B.Cu") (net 22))
 (segment (start 121.4252 117.645) (end 120.65 118.4202) (width 0.25) (layer "B.Cu") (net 22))
 (segment (start 105.41 143.4082) (end 105.41 155.3) (width 0.25) (layer "B.Cu") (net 22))
 (segment (start 135.0976 119.9609) (end 134.1251 119.9609) (width 0.25) (layer "B.Cu") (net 22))
 (segment (start 101.6 139.5982) (end 105.41 143.4082) (width 0.25) (layer "B.Cu") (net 22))
 (segment (start 132.5682 117.645) (end 121.4252 117.645) (width 0.25) (layer "B.Cu") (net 22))
 (segment (start 133.2069 119.0427) (end 133.2069 118.2837) (width 0.25) (layer "B.Cu") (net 22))
 (segment (start 120.65 119.8771) (end 101.6 138.9271) (width 0.25) (layer "B.Cu") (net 22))
 (segment (start 134.1251 119.9609) (end 133.2069 119.0427) (width 0.25) (layer "B.Cu") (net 22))
 (segment (start 148.5901 118.3761) (end 146.5102 116.2962) (width 0.25) (layer "B.Cu") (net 22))
 (segment (start 101.6 139.4405) (end 101.6 139.5982) (width 0.25) (layer "B.Cu") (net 22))
 (segment (start 133.2069 118.2837) (end 132.5682 117.645) (width 0.25) (layer "B.Cu") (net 22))
 (segment (start 101.6 139.4405) (end 101.6 138.9271) (width 0.25) (layer "B.Cu") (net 22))
 (segment (start 148.5901 119.1853) (end 148.5901 118.3761) (width 0.25) (layer "B.Cu") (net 22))
 (segment (start 137.9902 116.2962) (end 135.89 118.3964) (width 0.25) (layer "B.Cu") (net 22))
 (segment (start 120.65 118.4202) (end 120.65 119.8771) (width 0.25) (layer "B.Cu") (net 22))
 (segment (start 135.89 118.3964) (end 135.89 119.1685) (width 0.25) (layer "B.Cu") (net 22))
 (segment (start 96.52 163.068) (end 96.52 167.64) (width 0.25) (layer "F.Cu") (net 13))
 (segment (start 100.9489 158.6391) (end 96.52 163.068) (width 0.25) (layer "B.Cu") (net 13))
 (segment (start 137.165 159.766) (end 136.0381 158.6391) (width 0.25) (layer "B.Cu") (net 13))
 (segment (start 136.0381 158.6391) (end 100.9489 158.6391) (width 0.25) (layer "B.Cu") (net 13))
 (segment (start 118.6732 167.64) (end 125.5919 160.7213) (width 0.25) (layer "F.Cu") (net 14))
 (segment (start 143.51 118.4356) (end 143.51 119.1784) (width 0.25) (layer "F.Cu") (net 14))
 (segment (start 125.5919 159.5339) (end 132.9848 152.141) (width 0.25) (layer "F.Cu") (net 14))
 (segment (start 135.772 119.9478) (end 134.62 118.7958) (width 0.25) (layer "F.Cu") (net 14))
 (segment (start 143.51 119.1784) (end 142.7406 119.9478) (width 0.25) (layer "F.Cu") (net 14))
 (segment (start 178.6763 117.2083) (end 144.7373 117.2083) (width 0.25) (layer "F.Cu") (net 14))
 (segment (start 185.674 124.206) (end 178.6763 117.2083) (width 0.25) (layer "F.Cu") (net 14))
 (segment (start 144.7373 117.2083) (end 143.51 118.4356) (width 0.25) (layer "F.Cu") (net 14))
 (segment (start 142.7406 119.9478) (end 135.772 119.9478) (width 0.25) (layer "F.Cu") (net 14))
 (segment (start 101.6 167.64) (end 118.6732 167.64) (width 0.25) (layer "F.Cu") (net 14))
 (segment (start 135.772 150.989) (end 134.62 152.141) (width 0.25) (layer "F.Cu") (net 14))
 (segment (start 132.9848 152.141) (end 134.62 152.141) (width 0.25) (layer "F.Cu") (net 14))
 (segment (start 135.772 119.9478) (end 135.772 150.989) (width 0.25) (layer "F.Cu") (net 14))
 (segment (start 125.5919 160.7213) (end 125.5919 159.5339) (width 0.25) (layer "F.Cu") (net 14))
 (segment (start 134.62 152.141) (end 142.245 159.766) (width 0.25) (layer "F.Cu") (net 14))
 (segment (start 132.992 117.1678) (end 119.313 117.1678) (width 0.25) (layer "B.Cu") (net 14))
 (segment (start 117.9669 118.5139) (end 117.9669 118.7958) (width 0.25) (layer "B.Cu") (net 14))
 (segment (start 119.313 117.1678) (end 117.9669 118.5139) (width 0.25) (layer "B.Cu") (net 14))
 (segment (start 116.84 118.7958) (end 117.9669 118.7958) (width 0.25) (layer "B.Cu") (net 14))
 (segment (start 134.62 118.7958) (end 132.992 117.1678) (width 0.25) (layer "B.Cu") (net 14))
 (segment (start 138.5392 117.635) (end 133.2408 117.635) (width 0.25) (layer "F.Cu") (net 26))
 (segment (start 139.7 118.7958) (end 138.5392 117.635) (width 0.25) (layer "F.Cu") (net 26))
 (segment (start 133.2408 117.635) (end 132.08 118.7958) (width 0.25) (layer "F.Cu") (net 26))
 (segment (start 181.7233 149.0606) (end 181.7233 149.8) (width 0.25) (layer "B.Cu") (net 26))
 (segment (start 184.404 151.8113) (end 184.404 152.4807) (width 0.25) (layer "B.Cu") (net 26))
 (segment (start 141.2896 117.2062) (end 144.8362 117.2062) (width 0.25) (layer "B.Cu") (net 26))
 (segment (start 144.8362 117.2062) (end 145.9069 118.2769) (width 0.25) (layer "B.Cu") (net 26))
 (segment (start 182.7993 150.876) (end 183.4687 150.876) (width 0.25) (layer "B.Cu") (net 26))
 (segment (start 165.0945 138.176) (end 170.8387 138.176) (width 0.25) (layer "B.Cu") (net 26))
 (segment (start 183.4687 150.876) (end 184.404 151.8113) (width 0.25) (layer "B.Cu") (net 26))
 (segment (start 170.8387 138.176) (end 181.7233 149.0606) (width 0.25) (layer "B.Cu") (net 26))
 (segment (start 145.9069 118.2769) (end 145.9069 118.9884) (width 0.25) (layer "B.Cu") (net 26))
 (segment (start 145.9069 118.9884) (end 165.0945 138.176) (width 0.25) (layer "B.Cu") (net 26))
 (segment (start 181.7233 149.8) (end 182.7993 150.876) (width 0.25) (layer "B.Cu") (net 26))
 (segment (start 139.7 118.7958) (end 141.2896 117.2062) (width 0.25) (layer "B.Cu") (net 26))
 (segment (start 185.3393 153.416) (end 186.0608 153.416) (width 0.25) (layer "B.Cu") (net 26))
 (segment (start 186.0608 153.416) (end 186.825 154.1802) (width 0.25) (layer "B.Cu") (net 26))
 (segment (start 186.825 154.1802) (end 186.825 156.075) (width 0.25) (layer "B.Cu") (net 26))
 (segment (start 186.825 156.075) (end 185.674 157.226) (width 0.25) (layer "B.Cu") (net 26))
 (segment (start 184.404 152.4807) (end 185.3393 153.416) (width 0.25) (layer "B.Cu") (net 26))
 (segment (start 170.434 157.226) (end 167.8056 154.5976) (width 0.25) (layer "F.Cu") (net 27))
 (segment (start 167.8056 139.2814) (end 147.32 118.7958) (width 0.25) (layer "F.Cu") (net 27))
 (segment (start 167.8056 154.5976) (end 167.8056 139.2814) (width 0.25) (layer "F.Cu") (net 27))
 (segment (start 137.16 118.7958) (end 139.204 116.7518) (width 0.25) (layer "B.Cu") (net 27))
 (segment (start 145.276 116.7518) (end 147.32 118.7958) (width 0.25) (layer "B.Cu") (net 27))
 (segment (start 139.204 116.7518) (end 145.276 116.7518) (width 0.25) (layer "B.Cu") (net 27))
 (segment (start 181.864 151.7767) (end 180.9633 150.876) (width 0.25) (layer "B.Cu") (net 23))
 (segment (start 184.0173 154.686) (end 181.864 152.5327) (width 0.25) (layer "B.Cu") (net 23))
 (segment (start 180.9633 150.876) (end 154.0002 150.876) (width 0.25) (layer "B.Cu") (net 23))
 (segment (start 154.0002 150.876) (end 121.92 118.7958) (width 0.25) (layer "B.Cu") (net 23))
 (segment (start 181.864 152.5327) (end 181.864 151.7767) (width 0.25) (layer "B.Cu") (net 23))
 (segment (start 185.674 154.686) (end 184.0173 154.686) (width 0.25) (layer "B.Cu") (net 23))
 (segment (start 187.3128 123.6114) (end 156.6024 92.901) (width 0.25) (layer "B.Cu") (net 7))
 (segment (start 156.6024 92.901) (end 138.875 92.901) (width 0.25) (layer "B.Cu") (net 7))
 (segment (start 187.3128 142.8872) (end 187.3128 123.6114) (width 0.25) (layer "B.Cu") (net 7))
 (segment (start 138.875 92.901) (end 134.366 88.392) (width 0.25) (layer "B.Cu") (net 7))
 (segment (start 185.674 144.526) (end 187.3128 142.8872) (width 0.25) (layer "B.Cu") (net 7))
 (segment (start 185.674 141.986) (end 171.704 128.016) (width 0.25) (layer "B.Cu") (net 8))
 (segment (start 131.826 89.7416) (end 131.826 88.392) (width 0.25) (layer "B.Cu") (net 8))
 (segment (start 171.704 128.016) (end 170.1004 128.016) (width 0.25) (layer "B.Cu") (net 8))
 (segment (start 170.1004 128.016) (end 131.826 89.7416) (width 0.25) (layer "B.Cu") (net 8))
 (segment (start 144.78 118.7958) (end 145.911 117.6648) (width 0.25) (layer "F.Cu") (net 25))
 (segment (start 150.3663 117.6648) (end 169.3071 136.6056) (width 0.25) (layer "F.Cu") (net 25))
 (segment (start 145.911 117.6648) (end 150.3663 117.6648) (width 0.25) (layer "F.Cu") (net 25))
 (segment (start 169.3071 136.6056) (end 169.3071 153.5591) (width 0.25) (layer "F.Cu") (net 25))
 (segment (start 169.3071 153.5591) (end 170.434 154.686) (width 0.25) (layer "F.Cu") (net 25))
 (segment (start 140.97 118.3964) (end 141.7022 117.6642) (width 0.25) (layer "B.Cu") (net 25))
 (segment (start 143.6484 117.6642) (end 144.78 118.7958) (width 0.25) (layer "B.Cu") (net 25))
 (segment (start 131.1967 120.4525) (end 139.6504 120.4525) (width 0.25) (layer "B.Cu") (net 25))
 (segment (start 141.7022 117.6642) (end 143.6484 117.6642) (width 0.25) (layer "B.Cu") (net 25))
 (segment (start 139.6504 120.4525) (end 140.97 119.1329) (width 0.25) (layer "B.Cu") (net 25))
 (segment (start 129.54 118.7958) (end 131.1967 120.4525) (width 0.25) (layer "B.Cu") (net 25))
 (segment (start 140.97 119.1329) (end 140.97 118.3964) (width 0.25) (layer "B.Cu") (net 25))
 (segment (start 129.5206 121.3164) (end 142.1444 121.3164) (width 0.25) (layer "B.Cu") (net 24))
 (segment (start 142.1444 121.3164) (end 170.434 149.606) (width 0.25) (layer "B.Cu") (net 24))
 (segment (start 127 118.7958) (end 129.5206 121.3164) (width 0.25) (layer "B.Cu") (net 24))
 (segment (start 162.8902 139.446) (end 142.24 118.7958) (width 0.25) (layer "B.Cu") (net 28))
 (segment (start 170.434 139.446) (end 162.8902 139.446) (width 0.25) (layer "B.Cu") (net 28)))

